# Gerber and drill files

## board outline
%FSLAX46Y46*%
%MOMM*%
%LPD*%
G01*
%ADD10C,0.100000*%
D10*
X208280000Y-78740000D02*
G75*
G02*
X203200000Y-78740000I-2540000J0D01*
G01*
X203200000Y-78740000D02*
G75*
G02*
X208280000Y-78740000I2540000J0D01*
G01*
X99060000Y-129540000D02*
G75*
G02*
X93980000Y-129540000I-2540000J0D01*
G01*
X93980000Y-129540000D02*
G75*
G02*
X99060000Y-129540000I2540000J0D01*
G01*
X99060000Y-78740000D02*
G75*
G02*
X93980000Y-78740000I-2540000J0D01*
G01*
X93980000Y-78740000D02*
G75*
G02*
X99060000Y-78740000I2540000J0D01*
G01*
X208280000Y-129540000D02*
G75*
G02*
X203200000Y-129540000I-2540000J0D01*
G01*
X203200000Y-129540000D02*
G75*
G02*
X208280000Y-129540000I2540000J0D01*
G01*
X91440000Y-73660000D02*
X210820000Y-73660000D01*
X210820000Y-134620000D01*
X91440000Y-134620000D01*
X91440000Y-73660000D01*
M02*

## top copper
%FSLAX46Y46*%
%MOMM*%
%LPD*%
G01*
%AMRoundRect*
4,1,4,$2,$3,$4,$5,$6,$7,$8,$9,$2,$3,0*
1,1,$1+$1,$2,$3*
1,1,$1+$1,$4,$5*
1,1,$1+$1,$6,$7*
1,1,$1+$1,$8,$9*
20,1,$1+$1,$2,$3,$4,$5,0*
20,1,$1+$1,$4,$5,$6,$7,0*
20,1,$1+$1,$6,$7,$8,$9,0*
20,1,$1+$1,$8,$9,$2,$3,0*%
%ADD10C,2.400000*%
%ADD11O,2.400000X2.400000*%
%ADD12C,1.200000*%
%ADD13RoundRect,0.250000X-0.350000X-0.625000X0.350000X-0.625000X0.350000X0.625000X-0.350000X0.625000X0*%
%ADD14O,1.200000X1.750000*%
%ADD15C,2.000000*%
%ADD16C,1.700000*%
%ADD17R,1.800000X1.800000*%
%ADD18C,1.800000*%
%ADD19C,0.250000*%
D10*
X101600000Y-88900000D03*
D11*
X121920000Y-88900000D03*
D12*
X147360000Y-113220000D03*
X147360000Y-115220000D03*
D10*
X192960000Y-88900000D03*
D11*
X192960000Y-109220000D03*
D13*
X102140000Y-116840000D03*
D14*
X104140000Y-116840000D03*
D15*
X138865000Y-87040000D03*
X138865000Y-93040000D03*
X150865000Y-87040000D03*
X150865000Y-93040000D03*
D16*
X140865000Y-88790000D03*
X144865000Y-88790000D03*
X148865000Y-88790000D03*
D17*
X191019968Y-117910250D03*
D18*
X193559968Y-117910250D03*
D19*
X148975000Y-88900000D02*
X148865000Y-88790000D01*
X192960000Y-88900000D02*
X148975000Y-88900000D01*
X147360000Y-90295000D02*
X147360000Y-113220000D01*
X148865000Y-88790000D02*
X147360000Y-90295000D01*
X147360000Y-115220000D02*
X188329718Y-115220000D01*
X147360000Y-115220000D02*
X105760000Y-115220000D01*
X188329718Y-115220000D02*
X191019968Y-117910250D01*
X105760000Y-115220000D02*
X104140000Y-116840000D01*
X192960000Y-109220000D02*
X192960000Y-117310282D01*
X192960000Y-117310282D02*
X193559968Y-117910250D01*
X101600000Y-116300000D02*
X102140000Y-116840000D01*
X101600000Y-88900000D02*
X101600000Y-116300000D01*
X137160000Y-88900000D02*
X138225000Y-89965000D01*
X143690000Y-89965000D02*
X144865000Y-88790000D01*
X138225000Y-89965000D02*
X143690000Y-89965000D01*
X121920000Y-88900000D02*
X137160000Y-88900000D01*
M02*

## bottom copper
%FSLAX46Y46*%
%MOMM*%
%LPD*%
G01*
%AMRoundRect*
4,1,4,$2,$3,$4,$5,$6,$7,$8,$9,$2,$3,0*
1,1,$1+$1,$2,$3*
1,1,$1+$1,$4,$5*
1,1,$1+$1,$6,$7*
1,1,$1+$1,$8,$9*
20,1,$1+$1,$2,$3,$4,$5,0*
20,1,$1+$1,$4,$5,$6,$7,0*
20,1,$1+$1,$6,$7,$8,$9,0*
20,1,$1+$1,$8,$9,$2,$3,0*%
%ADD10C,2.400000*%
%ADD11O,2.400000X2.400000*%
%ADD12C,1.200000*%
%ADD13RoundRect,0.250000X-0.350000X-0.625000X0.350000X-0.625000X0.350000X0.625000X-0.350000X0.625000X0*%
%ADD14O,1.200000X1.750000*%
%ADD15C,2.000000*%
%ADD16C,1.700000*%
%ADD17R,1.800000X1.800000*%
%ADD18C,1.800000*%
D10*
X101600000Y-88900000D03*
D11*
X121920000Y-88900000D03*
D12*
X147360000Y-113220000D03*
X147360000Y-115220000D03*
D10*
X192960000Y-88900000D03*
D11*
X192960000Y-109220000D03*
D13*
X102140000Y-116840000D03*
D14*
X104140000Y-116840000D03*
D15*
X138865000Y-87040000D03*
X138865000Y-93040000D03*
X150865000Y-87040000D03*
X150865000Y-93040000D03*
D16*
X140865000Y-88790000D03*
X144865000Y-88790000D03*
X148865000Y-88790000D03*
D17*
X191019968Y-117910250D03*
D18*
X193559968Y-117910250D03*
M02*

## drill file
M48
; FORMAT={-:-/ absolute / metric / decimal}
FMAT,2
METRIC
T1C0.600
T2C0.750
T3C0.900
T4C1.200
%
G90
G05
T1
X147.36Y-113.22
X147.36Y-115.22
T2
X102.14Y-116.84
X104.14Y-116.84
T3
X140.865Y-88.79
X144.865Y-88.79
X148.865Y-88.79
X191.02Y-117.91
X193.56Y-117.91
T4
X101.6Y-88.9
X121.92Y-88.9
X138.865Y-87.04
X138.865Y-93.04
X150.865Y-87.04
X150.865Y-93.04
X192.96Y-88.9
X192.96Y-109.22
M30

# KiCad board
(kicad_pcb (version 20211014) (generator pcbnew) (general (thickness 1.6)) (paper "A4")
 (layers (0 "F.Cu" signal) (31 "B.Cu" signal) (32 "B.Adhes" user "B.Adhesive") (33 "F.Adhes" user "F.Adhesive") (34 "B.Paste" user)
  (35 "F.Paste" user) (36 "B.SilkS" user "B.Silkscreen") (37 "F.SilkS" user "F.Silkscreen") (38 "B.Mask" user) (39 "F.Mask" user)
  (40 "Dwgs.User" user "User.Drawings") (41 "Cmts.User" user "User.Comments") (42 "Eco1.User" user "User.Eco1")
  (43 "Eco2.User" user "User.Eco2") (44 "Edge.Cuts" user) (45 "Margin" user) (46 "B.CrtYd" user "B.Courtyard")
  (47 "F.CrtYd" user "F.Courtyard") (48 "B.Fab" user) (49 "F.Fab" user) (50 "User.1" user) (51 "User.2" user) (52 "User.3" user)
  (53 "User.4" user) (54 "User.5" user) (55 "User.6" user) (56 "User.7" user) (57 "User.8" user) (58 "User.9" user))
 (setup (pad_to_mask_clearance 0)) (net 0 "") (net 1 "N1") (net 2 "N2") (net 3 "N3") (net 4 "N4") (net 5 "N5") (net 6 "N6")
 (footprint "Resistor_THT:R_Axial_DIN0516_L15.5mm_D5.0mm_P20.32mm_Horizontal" (layer "F.Cu") (at 101.6 88.9)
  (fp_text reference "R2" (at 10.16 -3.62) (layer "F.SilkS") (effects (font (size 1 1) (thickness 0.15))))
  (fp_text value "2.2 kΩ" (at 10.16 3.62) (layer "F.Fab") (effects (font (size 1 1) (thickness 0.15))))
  (pad "1" thru_hole circle (at 0 0) (size 2.4 2.4) (drill 1.2) (layers *.Cu *.Mask) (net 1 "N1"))
  (pad "2" thru_hole oval (at 20.32 0) (size 2.4 2.4) (drill 1.2) (layers *.Cu *.Mask) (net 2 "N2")))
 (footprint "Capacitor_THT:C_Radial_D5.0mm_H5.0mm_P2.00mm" (layer "F.Cu") (at 147.36 113.22 -90)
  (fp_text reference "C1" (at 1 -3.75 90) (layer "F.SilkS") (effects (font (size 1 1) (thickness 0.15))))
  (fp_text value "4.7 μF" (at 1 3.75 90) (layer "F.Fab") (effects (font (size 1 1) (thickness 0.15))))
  (pad "1" thru_hole circle (at 0 0 270) (size 1.2 1.2) (drill 0.6) (layers *.Cu *.Mask) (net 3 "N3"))
  (pad "2" thru_hole circle (at 2 0 270) (size 1.2 1.2) (drill 0.6) (layers *.Cu *.Mask) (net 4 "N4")))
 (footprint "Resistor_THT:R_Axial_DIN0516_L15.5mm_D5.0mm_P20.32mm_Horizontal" (layer "F.Cu") (at 192.96 88.9 -90)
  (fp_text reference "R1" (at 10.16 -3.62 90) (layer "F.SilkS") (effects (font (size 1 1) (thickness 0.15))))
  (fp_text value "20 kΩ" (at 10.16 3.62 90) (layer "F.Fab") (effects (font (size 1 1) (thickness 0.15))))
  (pad "1" thru_hole circle (at 0 0 270) (size 2.4 2.4) (drill 1.2) (layers *.Cu *.Mask) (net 3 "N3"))
  (pad "2" thru_hole oval (at 20.32 0 270) (size 2.4 2.4) (drill 1.2) (layers *.Cu *.Mask) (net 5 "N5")))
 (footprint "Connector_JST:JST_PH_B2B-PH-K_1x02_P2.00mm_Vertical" (layer "F.Cu") (at 102.14 116.84)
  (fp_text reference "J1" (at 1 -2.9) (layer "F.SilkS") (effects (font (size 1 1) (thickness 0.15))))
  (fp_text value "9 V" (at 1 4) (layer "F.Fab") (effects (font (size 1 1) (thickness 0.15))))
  (pad "1" thru_hole roundrect (at 0 0) (size 1.2 1.75) (drill 0.75) (layers *.Cu *.Mask) (roundrect_rratio 0.2083333333) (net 1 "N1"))
  (pad "2" thru_hole oval (at 2 0) (size 1.2 1.75) (drill 0.75) (layers *.Cu *.Mask) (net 4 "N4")))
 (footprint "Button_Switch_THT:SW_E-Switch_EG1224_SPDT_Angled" (layer "F.Cu") (at 140.865 88.79)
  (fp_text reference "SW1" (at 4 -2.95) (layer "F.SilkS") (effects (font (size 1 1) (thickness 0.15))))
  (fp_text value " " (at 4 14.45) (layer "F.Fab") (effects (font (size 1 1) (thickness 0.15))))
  (pad "" thru_hole circle (at -2 -1.75) (size 2 2) (drill 1.2) (layers *.Cu *.Mask))
  (pad "" thru_hole circle (at -2 4.25) (size 2 2) (drill 1.2) (layers *.Cu *.Mask))
  (pad "" thru_hole circle (at 10 -1.75) (size 2 2) (drill 1.2) (layers *.Cu *.Mask))
  (pad "" thru_hole circle (at 10 4.25) (size 2 2) (drill 1.2) (layers *.Cu *.Mask))
  (pad "1" thru_hole circle (at 0 0) (size 1.7 1.7) (drill 0.9) (layers *.Cu *.Mask) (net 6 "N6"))
  (pad "2" thru_hole circle (at 4 0) (size 1.7 1.7) (drill 0.9) (layers *.Cu *.Mask) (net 2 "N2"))
  (pad "3" thru_hole circle (at 8 0) (size 1.7 1.7) (drill 0.9) (layers *.Cu *.Mask) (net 3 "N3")))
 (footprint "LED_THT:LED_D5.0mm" (layer "F.Cu") (at 191.019968 117.91025)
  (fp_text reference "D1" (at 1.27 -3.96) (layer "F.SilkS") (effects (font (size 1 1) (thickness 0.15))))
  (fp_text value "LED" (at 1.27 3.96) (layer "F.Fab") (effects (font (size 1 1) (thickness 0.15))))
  (pad "1" thru_hole rect (at 0 0) (size 1.8 1.8) (drill 0.9) (layers *.Cu *.Mask) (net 4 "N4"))
  (pad "2" thru_hole circle (at 2.54 0) (size 1.8 1.8) (drill 0.9) (layers *.Cu *.Mask) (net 5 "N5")))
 (gr_circle (center 205.74 78.74) (end 208.28 78.74) (layer "Edge.Cuts") (width 0.1) (fill none))
 (gr_circle (center 96.52 129.54) (end 99.06 129.54) (layer "Edge.Cuts") (width 0.1) (fill none))
 (gr_circle (center 96.52 78.74) (end 99.06 78.74) (layer "Edge.Cuts") (width 0.1) (fill none))
 (gr_circle (center 205.74 129.54) (end 208.28 129.54) (layer "Edge.Cuts") (width 0.1) (fill none))
 (gr_rect (start 91.44 73.66) (end 210.82 134.62) (layer "Edge.Cuts") (width 0.1) (fill none))
 (segment (start 148.975 88.9) (end 148.865 88.79) (width 0.25) (layer "F.Cu") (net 3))
 (segment (start 192.96 88.9) (end 148.975 88.9) (width 0.25) (layer "F.Cu") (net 3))
 (segment (start 147.36 90.295) (end 147.36 113.22) (width 0.25) (layer "F.Cu") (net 3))
 (segment (start 148.865 88.79) (end 147.36 90.295) (width 0.25) (layer "F.Cu") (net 3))
 (segment (start 147.36 115.22) (end 188.329718 115.22) (width 0.25) (layer "F.Cu") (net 4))
 (segment (start 147.36 115.22) (end 105.76 115.22) (width 0.25) (layer "F.Cu") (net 4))
 (segment (start 188.329718 115.22) (end 191.019968 117.91025) (width 0.25) (layer "F.Cu") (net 4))
 (segment (start 105.76 115.22) (end 104.14 116.84) (width 0.25) (layer "F.Cu") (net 4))
 (segment (start 192.96 109.22) (end 192.96 117.310282) (width 0.25) (layer "F.Cu") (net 5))
 (segment (start 192.96 117.310282) (end 193.559968 117.91025) (width 0.25) (layer "F.Cu") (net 5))
 (segment (start 101.6 116.3) (end 102.14 116.84) (width 0.25) (layer "F.Cu") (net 1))
 (segment (start 101.6 88.9) (end 101.6 116.3) (width 0.25) (layer "F.Cu") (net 1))
 (segment (start 137.16 88.9) (end 138.225 89.965) (width 0.25) (layer "F.Cu") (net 2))
 (segment (start 143.69 89.965) (end 144.865 88.79) (width 0.25) (layer "F.Cu") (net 2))
 (segment (start 138.225 89.965) (end 143.69 89.965) (width 0.25) (layer "F.Cu") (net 2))
 (segment (start 121.92 88.9) (end 137.16 88.9) (width 0.25) (layer "F.Cu") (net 2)))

